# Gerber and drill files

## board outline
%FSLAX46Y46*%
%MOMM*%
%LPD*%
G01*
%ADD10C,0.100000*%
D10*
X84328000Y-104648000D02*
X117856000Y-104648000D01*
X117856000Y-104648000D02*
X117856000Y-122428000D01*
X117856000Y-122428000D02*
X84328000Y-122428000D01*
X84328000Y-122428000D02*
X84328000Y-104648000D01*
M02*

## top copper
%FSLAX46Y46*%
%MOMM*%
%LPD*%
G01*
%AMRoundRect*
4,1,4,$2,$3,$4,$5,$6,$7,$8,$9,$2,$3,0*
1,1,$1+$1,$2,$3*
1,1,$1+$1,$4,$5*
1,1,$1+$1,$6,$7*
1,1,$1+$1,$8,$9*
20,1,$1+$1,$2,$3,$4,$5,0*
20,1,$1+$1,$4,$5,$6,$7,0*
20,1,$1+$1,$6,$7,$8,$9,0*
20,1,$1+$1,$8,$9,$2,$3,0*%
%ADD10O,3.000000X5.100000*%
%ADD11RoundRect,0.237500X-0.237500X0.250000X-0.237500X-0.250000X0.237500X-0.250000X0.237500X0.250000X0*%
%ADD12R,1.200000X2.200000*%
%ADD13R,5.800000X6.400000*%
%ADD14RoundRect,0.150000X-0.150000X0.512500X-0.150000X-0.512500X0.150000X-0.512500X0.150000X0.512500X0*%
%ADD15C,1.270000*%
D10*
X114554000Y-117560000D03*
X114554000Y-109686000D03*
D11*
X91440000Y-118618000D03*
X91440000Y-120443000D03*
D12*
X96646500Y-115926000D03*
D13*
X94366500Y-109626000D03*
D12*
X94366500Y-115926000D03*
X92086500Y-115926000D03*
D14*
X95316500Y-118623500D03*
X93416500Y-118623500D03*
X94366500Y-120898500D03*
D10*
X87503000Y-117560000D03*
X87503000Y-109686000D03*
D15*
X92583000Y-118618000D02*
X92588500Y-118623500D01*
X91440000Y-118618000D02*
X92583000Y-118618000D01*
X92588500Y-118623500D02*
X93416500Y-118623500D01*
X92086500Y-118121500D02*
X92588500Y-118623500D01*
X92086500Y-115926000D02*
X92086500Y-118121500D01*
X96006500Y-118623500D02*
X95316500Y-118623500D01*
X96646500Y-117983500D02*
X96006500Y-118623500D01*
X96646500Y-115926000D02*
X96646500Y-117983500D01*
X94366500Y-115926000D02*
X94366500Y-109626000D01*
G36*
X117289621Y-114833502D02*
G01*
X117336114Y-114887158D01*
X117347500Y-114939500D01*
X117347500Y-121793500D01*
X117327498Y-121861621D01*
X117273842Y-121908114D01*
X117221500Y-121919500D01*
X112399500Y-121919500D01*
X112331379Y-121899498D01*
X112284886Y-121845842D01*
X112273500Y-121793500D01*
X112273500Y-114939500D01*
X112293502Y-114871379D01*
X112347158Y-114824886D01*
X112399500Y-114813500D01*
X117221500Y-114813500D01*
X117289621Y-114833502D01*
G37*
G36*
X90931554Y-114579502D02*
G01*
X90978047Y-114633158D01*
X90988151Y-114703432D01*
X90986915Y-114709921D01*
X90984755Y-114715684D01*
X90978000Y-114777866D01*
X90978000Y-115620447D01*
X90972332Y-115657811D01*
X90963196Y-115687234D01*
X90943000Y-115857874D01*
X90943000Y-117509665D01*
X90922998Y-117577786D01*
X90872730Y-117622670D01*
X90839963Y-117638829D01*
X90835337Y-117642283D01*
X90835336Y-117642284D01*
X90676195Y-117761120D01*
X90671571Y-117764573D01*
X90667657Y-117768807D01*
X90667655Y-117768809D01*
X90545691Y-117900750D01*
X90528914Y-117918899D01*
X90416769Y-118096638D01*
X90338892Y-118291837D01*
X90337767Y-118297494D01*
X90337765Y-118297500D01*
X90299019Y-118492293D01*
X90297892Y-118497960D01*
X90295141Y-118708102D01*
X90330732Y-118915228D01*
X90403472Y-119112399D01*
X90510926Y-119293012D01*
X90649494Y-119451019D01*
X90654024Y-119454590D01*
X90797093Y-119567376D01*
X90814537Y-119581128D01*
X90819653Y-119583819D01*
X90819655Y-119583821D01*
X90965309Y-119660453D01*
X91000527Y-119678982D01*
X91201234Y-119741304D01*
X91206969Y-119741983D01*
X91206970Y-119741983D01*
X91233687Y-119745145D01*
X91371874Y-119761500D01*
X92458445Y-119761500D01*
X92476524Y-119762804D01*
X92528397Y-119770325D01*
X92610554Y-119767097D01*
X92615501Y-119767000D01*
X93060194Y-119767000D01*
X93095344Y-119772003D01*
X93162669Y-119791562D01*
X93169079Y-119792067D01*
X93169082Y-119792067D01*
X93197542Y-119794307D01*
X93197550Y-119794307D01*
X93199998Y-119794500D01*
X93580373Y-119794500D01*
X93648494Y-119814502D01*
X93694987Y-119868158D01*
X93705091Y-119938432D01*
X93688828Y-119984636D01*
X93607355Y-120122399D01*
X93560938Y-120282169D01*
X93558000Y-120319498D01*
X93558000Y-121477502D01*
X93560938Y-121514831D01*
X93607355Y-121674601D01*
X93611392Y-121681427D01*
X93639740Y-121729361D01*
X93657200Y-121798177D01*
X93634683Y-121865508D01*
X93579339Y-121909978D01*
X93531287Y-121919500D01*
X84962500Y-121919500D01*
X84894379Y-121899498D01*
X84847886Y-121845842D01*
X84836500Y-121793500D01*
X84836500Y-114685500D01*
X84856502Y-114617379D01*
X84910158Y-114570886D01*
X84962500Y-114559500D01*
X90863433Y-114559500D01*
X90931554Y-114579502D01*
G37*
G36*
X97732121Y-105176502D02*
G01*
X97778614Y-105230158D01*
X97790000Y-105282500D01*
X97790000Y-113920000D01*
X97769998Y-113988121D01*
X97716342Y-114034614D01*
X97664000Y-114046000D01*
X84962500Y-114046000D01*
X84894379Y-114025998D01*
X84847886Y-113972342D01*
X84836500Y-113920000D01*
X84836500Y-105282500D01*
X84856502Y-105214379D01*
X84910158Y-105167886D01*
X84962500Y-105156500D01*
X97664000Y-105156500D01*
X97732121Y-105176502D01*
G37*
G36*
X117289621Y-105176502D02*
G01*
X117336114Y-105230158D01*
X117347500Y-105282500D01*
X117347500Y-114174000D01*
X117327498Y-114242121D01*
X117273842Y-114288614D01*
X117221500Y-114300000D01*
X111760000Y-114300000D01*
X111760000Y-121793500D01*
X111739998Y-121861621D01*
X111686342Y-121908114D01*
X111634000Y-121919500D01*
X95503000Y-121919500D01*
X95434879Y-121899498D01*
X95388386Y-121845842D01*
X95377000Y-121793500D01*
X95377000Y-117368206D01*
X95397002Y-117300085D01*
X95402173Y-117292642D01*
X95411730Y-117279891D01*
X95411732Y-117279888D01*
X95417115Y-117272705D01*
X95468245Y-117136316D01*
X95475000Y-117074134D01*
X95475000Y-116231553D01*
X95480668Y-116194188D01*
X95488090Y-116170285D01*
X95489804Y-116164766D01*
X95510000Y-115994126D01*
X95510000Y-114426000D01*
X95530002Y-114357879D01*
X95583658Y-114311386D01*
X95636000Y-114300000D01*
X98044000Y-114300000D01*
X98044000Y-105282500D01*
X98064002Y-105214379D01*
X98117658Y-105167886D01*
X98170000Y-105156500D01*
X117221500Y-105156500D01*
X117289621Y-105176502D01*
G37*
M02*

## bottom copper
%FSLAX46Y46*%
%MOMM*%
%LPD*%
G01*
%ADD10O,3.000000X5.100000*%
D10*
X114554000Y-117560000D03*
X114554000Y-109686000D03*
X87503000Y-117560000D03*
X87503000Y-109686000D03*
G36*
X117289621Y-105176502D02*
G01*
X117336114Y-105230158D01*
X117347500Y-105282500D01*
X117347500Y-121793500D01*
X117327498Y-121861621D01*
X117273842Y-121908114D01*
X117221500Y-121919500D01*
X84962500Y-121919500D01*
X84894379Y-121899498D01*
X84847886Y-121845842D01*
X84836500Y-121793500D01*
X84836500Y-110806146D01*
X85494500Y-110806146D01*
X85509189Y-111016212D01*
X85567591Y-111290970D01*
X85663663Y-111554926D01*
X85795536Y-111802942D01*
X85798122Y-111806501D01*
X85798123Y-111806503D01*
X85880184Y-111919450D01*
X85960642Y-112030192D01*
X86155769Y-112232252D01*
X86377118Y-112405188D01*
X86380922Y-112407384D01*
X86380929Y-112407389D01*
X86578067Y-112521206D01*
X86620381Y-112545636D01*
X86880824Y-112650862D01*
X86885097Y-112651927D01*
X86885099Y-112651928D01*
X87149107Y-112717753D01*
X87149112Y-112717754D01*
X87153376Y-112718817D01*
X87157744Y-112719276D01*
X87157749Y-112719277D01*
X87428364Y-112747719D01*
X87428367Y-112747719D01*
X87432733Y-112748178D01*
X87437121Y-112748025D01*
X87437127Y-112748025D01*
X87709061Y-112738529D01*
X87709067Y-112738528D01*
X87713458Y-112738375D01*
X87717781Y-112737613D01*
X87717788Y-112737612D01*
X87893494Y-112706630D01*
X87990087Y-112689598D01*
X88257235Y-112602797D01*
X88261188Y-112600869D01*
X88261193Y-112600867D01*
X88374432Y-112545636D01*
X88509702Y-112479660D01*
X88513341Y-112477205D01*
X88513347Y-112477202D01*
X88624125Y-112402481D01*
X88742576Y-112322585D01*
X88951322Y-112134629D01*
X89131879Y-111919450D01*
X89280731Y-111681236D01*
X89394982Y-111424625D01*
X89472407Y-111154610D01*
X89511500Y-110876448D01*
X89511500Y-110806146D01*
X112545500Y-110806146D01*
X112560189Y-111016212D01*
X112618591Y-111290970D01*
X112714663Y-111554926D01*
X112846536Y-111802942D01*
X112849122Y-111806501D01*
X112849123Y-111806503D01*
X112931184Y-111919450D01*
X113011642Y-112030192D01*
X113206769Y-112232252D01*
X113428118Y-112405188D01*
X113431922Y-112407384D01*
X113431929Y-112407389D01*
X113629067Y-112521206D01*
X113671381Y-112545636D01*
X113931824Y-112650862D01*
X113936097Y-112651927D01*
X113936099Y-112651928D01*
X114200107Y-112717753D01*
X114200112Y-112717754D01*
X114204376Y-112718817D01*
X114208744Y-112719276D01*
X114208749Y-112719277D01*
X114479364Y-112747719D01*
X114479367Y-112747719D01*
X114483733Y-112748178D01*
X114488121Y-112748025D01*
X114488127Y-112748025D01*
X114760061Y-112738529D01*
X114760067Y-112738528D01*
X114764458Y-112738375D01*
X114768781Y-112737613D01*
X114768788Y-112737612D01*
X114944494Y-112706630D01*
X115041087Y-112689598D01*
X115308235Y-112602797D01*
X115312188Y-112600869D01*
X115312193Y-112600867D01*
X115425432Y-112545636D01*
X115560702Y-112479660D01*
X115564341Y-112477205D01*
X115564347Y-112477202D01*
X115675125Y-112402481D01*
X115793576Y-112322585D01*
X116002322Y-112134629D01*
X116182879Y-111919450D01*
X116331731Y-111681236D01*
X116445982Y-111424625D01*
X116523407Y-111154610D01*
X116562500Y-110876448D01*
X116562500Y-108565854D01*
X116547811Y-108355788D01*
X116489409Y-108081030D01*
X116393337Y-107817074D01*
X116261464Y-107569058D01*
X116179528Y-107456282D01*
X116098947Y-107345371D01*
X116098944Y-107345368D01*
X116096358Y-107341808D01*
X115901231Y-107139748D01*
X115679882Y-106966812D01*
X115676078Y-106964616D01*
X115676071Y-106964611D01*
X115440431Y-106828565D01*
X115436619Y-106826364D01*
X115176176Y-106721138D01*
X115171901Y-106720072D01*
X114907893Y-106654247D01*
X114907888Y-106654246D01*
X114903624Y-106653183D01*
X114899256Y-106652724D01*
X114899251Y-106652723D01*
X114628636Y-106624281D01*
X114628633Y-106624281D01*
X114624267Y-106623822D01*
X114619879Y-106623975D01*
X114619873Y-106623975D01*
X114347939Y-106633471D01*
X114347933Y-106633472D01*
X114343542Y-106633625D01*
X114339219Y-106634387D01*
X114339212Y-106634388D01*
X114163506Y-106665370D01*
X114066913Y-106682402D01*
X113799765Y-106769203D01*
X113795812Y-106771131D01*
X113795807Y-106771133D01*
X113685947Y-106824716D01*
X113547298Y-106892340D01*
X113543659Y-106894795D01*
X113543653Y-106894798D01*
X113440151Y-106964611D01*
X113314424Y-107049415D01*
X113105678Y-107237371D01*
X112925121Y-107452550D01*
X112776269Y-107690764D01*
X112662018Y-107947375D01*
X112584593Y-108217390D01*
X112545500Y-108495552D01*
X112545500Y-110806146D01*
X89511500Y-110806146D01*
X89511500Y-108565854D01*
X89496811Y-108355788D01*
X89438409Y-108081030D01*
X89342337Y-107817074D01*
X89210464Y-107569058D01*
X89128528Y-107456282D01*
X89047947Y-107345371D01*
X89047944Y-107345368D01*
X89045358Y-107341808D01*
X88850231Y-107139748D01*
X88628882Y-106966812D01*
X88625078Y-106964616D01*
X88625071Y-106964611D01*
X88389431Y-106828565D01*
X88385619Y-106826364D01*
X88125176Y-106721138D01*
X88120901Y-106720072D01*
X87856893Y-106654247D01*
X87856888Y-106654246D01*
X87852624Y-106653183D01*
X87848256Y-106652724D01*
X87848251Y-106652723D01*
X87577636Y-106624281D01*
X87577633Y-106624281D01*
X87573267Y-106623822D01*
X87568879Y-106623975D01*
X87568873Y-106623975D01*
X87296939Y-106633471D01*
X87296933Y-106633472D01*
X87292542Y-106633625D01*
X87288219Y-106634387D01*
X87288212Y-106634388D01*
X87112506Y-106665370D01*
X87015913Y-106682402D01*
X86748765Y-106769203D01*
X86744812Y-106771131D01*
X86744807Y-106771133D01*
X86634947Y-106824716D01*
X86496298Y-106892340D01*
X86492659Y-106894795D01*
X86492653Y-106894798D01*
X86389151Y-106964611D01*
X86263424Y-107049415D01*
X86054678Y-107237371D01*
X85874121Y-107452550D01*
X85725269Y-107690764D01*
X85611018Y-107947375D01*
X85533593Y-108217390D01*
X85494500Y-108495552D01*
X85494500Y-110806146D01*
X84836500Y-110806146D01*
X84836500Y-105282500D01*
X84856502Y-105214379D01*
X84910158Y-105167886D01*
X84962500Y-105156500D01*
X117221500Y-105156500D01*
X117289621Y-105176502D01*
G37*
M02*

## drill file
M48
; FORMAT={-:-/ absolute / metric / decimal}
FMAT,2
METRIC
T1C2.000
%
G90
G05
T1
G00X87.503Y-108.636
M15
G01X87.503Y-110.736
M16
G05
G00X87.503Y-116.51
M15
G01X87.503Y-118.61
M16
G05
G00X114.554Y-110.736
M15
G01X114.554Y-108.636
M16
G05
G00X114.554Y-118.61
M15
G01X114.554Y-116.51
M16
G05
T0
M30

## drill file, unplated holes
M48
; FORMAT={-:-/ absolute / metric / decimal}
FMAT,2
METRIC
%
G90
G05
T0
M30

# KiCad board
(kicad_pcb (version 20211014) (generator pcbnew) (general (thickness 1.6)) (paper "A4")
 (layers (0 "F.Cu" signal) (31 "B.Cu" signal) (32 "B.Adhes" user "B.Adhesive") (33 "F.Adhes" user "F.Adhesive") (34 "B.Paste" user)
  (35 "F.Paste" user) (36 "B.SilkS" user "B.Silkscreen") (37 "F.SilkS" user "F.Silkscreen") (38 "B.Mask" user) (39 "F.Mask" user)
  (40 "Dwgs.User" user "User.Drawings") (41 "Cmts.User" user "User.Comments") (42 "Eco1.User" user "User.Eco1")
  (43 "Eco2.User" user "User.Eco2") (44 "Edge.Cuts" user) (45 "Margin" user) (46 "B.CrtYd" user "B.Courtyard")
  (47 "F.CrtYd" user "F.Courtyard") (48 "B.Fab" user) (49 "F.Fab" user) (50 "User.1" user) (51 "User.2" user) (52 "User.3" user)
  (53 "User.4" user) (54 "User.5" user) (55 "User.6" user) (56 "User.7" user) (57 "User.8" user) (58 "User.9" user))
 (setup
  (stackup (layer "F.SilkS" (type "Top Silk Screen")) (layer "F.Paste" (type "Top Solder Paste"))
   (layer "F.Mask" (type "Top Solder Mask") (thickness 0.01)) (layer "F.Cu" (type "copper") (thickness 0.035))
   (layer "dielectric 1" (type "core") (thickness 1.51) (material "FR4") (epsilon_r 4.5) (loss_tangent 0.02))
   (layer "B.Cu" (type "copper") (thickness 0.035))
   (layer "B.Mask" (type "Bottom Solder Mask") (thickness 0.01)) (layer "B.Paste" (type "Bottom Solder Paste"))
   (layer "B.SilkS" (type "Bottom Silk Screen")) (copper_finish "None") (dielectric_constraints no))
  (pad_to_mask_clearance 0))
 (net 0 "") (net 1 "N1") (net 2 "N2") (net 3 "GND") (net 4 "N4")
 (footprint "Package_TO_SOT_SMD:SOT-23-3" (layer "F.Cu") (at 94.3665 119.761 -90)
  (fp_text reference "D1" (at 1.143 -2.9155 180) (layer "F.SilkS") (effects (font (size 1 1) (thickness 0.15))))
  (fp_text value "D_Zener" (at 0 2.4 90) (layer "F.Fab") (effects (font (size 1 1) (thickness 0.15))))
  (pad "1" smd roundrect locked (at -1.1375 -0.95 270) (size 1.325 0.6) (layers "F.Cu" "F.Paste" "F.Mask") (roundrect_rratio 0.25)
   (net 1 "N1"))
  (pad "2" smd roundrect locked (at -1.1375 0.95 270) (size 1.325 0.6) (layers "F.Cu" "F.Paste" "F.Mask") (roundrect_rratio 0.25)
   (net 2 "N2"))
  (pad "3" smd roundrect locked (at 1.1375 0 270) (size 1.325 0.6) (layers "F.Cu" "F.Paste" "F.Mask") (roundrect_rratio 0.25)))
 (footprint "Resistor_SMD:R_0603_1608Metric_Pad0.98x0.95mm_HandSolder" (layer "F.Cu") (at 91.44 119.5305 -90)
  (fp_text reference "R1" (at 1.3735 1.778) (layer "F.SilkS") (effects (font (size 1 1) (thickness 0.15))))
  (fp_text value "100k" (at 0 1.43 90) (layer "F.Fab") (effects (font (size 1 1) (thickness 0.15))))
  (pad "1" smd roundrect (at -0.9125 0 270) (size 0.975 0.95) (layers "F.Cu" "F.Paste" "F.Mask") (roundrect_rratio 0.25) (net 2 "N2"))
  (pad "2" smd roundrect (at 0.9125 0 270) (size 0.975 0.95) (layers "F.Cu" "F.Paste" "F.Mask") (roundrect_rratio 0.25) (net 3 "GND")))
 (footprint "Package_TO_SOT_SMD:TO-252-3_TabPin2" (layer "F.Cu") (at 94.3665 111.726 90)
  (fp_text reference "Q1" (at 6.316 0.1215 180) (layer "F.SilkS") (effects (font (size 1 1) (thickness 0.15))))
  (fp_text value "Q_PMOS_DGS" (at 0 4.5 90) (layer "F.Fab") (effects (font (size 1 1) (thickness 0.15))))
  (pad "" smd rect (at 3.775 1.525 90) (size 3.05 2.75) (layers "F.Paste"))
  (pad "" smd rect (at 3.775 -1.525 90) (size 3.05 2.75) (layers "F.Paste"))
  (pad "" smd rect (at 0.425 -1.525 90) (size 3.05 2.75) (layers "F.Paste"))
  (pad "" smd rect (at 0.425 1.525 90) (size 3.05 2.75) (layers "F.Paste"))
  (pad "1" smd rect (at -4.2 -2.28 90) (size 2.2 1.2) (layers "F.Cu" "F.Paste" "F.Mask") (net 2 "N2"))
  (pad "2" smd rect (at -4.2 0 90) (size 2.2 1.2) (layers "F.Cu" "F.Paste" "F.Mask") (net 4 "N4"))
  (pad "2" smd rect (at 2.1 0 90) (size 6.4 5.8) (layers "F.Cu" "F.Mask") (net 4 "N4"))
  (pad "3" smd rect (at -4.2 2.28 90) (size 2.2 1.2) (layers "F.Cu" "F.Paste" "F.Mask") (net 1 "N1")))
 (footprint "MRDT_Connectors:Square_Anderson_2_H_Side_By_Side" (layer "F.Cu") (at 114.1794 118.11 180)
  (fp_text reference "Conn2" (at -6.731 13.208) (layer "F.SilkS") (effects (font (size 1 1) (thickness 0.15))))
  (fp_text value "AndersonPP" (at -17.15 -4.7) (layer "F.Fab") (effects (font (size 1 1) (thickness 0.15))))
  (pad "1" thru_hole oval locked (at -0.3746 0.55 180) (size 3 5.1) (drill oval 2 4.1) (layers *.Cu *.Mask "F.Paste") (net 3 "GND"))
  (pad "2" thru_hole oval locked (at -0.3746 8.424 180) (size 3 5.1) (drill oval 2 4.1) (layers *.Cu *.Mask "F.Paste") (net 1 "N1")))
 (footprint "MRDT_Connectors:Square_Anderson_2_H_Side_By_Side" (layer "B.Cu") (at 87.8776 118.11)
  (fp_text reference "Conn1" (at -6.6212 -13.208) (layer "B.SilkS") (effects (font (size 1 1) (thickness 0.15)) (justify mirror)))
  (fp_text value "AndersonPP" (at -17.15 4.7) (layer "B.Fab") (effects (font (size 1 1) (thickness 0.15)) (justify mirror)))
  (pad "1" thru_hole oval locked (at -0.3746 -0.55) (size 3 5.1) (drill oval 2 4.1) (layers *.Cu *.Mask "B.Paste") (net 3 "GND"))
  (pad "2" thru_hole oval locked (at -0.3746 -8.424) (size 3 5.1) (drill oval 2 4.1) (layers *.Cu *.Mask "B.Paste") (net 4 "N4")))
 (gr_rect (start 84.328 104.648) (end 117.856 122.428) (layer "Edge.Cuts") (width 0.1) (fill none))
 (segment (start 96.6465 117.9835) (end 96.0065 118.6235) (width 1.27) (layer "F.Cu") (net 1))
 (segment (start 96.0065 118.6235) (end 95.3165 118.6235) (width 1.27) (layer "F.Cu") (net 1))
 (segment (start 96.6465 115.926) (end 96.6465 117.9835) (width 1.27) (layer "F.Cu") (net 1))
 (segment (start 92.0865 118.1215) (end 92.5885 118.6235) (width 1.27) (layer "F.Cu") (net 2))
 (segment (start 92.583 118.618) (end 92.5885 118.6235) (width 1.27) (layer "F.Cu") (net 2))
 (segment (start 91.44 118.618) (end 92.583 118.618) (width 1.27) (layer "F.Cu") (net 2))
 (segment (start 92.0865 115.926) (end 92.0865 118.1215) (width 1.27) (layer "F.Cu") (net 2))
 (segment (start 92.5885 118.6235) (end 93.4165 118.6235) (width 1.27) (layer "F.Cu") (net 2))
 (segment (start 94.3665 115.926) (end 94.3665 109.626) (width 1.27) (layer "F.Cu") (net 4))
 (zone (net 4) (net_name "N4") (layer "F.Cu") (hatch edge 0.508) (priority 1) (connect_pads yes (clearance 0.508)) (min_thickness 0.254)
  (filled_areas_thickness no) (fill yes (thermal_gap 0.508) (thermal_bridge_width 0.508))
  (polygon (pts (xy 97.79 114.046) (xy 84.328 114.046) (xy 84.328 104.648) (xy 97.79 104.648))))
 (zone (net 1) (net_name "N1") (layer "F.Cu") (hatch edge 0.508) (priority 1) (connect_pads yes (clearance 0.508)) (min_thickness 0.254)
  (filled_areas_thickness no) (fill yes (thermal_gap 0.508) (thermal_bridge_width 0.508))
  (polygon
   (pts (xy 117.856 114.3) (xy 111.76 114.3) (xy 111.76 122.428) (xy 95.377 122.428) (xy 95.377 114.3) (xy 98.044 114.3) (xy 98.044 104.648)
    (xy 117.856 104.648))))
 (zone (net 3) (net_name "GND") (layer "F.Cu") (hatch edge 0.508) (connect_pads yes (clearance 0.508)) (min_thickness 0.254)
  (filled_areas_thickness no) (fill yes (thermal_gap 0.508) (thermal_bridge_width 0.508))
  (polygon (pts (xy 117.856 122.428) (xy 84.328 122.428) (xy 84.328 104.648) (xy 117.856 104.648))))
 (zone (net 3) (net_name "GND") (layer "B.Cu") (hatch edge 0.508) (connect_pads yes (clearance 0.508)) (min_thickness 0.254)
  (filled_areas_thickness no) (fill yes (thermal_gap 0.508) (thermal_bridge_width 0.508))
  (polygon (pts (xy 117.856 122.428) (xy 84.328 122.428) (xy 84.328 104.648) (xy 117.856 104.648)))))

